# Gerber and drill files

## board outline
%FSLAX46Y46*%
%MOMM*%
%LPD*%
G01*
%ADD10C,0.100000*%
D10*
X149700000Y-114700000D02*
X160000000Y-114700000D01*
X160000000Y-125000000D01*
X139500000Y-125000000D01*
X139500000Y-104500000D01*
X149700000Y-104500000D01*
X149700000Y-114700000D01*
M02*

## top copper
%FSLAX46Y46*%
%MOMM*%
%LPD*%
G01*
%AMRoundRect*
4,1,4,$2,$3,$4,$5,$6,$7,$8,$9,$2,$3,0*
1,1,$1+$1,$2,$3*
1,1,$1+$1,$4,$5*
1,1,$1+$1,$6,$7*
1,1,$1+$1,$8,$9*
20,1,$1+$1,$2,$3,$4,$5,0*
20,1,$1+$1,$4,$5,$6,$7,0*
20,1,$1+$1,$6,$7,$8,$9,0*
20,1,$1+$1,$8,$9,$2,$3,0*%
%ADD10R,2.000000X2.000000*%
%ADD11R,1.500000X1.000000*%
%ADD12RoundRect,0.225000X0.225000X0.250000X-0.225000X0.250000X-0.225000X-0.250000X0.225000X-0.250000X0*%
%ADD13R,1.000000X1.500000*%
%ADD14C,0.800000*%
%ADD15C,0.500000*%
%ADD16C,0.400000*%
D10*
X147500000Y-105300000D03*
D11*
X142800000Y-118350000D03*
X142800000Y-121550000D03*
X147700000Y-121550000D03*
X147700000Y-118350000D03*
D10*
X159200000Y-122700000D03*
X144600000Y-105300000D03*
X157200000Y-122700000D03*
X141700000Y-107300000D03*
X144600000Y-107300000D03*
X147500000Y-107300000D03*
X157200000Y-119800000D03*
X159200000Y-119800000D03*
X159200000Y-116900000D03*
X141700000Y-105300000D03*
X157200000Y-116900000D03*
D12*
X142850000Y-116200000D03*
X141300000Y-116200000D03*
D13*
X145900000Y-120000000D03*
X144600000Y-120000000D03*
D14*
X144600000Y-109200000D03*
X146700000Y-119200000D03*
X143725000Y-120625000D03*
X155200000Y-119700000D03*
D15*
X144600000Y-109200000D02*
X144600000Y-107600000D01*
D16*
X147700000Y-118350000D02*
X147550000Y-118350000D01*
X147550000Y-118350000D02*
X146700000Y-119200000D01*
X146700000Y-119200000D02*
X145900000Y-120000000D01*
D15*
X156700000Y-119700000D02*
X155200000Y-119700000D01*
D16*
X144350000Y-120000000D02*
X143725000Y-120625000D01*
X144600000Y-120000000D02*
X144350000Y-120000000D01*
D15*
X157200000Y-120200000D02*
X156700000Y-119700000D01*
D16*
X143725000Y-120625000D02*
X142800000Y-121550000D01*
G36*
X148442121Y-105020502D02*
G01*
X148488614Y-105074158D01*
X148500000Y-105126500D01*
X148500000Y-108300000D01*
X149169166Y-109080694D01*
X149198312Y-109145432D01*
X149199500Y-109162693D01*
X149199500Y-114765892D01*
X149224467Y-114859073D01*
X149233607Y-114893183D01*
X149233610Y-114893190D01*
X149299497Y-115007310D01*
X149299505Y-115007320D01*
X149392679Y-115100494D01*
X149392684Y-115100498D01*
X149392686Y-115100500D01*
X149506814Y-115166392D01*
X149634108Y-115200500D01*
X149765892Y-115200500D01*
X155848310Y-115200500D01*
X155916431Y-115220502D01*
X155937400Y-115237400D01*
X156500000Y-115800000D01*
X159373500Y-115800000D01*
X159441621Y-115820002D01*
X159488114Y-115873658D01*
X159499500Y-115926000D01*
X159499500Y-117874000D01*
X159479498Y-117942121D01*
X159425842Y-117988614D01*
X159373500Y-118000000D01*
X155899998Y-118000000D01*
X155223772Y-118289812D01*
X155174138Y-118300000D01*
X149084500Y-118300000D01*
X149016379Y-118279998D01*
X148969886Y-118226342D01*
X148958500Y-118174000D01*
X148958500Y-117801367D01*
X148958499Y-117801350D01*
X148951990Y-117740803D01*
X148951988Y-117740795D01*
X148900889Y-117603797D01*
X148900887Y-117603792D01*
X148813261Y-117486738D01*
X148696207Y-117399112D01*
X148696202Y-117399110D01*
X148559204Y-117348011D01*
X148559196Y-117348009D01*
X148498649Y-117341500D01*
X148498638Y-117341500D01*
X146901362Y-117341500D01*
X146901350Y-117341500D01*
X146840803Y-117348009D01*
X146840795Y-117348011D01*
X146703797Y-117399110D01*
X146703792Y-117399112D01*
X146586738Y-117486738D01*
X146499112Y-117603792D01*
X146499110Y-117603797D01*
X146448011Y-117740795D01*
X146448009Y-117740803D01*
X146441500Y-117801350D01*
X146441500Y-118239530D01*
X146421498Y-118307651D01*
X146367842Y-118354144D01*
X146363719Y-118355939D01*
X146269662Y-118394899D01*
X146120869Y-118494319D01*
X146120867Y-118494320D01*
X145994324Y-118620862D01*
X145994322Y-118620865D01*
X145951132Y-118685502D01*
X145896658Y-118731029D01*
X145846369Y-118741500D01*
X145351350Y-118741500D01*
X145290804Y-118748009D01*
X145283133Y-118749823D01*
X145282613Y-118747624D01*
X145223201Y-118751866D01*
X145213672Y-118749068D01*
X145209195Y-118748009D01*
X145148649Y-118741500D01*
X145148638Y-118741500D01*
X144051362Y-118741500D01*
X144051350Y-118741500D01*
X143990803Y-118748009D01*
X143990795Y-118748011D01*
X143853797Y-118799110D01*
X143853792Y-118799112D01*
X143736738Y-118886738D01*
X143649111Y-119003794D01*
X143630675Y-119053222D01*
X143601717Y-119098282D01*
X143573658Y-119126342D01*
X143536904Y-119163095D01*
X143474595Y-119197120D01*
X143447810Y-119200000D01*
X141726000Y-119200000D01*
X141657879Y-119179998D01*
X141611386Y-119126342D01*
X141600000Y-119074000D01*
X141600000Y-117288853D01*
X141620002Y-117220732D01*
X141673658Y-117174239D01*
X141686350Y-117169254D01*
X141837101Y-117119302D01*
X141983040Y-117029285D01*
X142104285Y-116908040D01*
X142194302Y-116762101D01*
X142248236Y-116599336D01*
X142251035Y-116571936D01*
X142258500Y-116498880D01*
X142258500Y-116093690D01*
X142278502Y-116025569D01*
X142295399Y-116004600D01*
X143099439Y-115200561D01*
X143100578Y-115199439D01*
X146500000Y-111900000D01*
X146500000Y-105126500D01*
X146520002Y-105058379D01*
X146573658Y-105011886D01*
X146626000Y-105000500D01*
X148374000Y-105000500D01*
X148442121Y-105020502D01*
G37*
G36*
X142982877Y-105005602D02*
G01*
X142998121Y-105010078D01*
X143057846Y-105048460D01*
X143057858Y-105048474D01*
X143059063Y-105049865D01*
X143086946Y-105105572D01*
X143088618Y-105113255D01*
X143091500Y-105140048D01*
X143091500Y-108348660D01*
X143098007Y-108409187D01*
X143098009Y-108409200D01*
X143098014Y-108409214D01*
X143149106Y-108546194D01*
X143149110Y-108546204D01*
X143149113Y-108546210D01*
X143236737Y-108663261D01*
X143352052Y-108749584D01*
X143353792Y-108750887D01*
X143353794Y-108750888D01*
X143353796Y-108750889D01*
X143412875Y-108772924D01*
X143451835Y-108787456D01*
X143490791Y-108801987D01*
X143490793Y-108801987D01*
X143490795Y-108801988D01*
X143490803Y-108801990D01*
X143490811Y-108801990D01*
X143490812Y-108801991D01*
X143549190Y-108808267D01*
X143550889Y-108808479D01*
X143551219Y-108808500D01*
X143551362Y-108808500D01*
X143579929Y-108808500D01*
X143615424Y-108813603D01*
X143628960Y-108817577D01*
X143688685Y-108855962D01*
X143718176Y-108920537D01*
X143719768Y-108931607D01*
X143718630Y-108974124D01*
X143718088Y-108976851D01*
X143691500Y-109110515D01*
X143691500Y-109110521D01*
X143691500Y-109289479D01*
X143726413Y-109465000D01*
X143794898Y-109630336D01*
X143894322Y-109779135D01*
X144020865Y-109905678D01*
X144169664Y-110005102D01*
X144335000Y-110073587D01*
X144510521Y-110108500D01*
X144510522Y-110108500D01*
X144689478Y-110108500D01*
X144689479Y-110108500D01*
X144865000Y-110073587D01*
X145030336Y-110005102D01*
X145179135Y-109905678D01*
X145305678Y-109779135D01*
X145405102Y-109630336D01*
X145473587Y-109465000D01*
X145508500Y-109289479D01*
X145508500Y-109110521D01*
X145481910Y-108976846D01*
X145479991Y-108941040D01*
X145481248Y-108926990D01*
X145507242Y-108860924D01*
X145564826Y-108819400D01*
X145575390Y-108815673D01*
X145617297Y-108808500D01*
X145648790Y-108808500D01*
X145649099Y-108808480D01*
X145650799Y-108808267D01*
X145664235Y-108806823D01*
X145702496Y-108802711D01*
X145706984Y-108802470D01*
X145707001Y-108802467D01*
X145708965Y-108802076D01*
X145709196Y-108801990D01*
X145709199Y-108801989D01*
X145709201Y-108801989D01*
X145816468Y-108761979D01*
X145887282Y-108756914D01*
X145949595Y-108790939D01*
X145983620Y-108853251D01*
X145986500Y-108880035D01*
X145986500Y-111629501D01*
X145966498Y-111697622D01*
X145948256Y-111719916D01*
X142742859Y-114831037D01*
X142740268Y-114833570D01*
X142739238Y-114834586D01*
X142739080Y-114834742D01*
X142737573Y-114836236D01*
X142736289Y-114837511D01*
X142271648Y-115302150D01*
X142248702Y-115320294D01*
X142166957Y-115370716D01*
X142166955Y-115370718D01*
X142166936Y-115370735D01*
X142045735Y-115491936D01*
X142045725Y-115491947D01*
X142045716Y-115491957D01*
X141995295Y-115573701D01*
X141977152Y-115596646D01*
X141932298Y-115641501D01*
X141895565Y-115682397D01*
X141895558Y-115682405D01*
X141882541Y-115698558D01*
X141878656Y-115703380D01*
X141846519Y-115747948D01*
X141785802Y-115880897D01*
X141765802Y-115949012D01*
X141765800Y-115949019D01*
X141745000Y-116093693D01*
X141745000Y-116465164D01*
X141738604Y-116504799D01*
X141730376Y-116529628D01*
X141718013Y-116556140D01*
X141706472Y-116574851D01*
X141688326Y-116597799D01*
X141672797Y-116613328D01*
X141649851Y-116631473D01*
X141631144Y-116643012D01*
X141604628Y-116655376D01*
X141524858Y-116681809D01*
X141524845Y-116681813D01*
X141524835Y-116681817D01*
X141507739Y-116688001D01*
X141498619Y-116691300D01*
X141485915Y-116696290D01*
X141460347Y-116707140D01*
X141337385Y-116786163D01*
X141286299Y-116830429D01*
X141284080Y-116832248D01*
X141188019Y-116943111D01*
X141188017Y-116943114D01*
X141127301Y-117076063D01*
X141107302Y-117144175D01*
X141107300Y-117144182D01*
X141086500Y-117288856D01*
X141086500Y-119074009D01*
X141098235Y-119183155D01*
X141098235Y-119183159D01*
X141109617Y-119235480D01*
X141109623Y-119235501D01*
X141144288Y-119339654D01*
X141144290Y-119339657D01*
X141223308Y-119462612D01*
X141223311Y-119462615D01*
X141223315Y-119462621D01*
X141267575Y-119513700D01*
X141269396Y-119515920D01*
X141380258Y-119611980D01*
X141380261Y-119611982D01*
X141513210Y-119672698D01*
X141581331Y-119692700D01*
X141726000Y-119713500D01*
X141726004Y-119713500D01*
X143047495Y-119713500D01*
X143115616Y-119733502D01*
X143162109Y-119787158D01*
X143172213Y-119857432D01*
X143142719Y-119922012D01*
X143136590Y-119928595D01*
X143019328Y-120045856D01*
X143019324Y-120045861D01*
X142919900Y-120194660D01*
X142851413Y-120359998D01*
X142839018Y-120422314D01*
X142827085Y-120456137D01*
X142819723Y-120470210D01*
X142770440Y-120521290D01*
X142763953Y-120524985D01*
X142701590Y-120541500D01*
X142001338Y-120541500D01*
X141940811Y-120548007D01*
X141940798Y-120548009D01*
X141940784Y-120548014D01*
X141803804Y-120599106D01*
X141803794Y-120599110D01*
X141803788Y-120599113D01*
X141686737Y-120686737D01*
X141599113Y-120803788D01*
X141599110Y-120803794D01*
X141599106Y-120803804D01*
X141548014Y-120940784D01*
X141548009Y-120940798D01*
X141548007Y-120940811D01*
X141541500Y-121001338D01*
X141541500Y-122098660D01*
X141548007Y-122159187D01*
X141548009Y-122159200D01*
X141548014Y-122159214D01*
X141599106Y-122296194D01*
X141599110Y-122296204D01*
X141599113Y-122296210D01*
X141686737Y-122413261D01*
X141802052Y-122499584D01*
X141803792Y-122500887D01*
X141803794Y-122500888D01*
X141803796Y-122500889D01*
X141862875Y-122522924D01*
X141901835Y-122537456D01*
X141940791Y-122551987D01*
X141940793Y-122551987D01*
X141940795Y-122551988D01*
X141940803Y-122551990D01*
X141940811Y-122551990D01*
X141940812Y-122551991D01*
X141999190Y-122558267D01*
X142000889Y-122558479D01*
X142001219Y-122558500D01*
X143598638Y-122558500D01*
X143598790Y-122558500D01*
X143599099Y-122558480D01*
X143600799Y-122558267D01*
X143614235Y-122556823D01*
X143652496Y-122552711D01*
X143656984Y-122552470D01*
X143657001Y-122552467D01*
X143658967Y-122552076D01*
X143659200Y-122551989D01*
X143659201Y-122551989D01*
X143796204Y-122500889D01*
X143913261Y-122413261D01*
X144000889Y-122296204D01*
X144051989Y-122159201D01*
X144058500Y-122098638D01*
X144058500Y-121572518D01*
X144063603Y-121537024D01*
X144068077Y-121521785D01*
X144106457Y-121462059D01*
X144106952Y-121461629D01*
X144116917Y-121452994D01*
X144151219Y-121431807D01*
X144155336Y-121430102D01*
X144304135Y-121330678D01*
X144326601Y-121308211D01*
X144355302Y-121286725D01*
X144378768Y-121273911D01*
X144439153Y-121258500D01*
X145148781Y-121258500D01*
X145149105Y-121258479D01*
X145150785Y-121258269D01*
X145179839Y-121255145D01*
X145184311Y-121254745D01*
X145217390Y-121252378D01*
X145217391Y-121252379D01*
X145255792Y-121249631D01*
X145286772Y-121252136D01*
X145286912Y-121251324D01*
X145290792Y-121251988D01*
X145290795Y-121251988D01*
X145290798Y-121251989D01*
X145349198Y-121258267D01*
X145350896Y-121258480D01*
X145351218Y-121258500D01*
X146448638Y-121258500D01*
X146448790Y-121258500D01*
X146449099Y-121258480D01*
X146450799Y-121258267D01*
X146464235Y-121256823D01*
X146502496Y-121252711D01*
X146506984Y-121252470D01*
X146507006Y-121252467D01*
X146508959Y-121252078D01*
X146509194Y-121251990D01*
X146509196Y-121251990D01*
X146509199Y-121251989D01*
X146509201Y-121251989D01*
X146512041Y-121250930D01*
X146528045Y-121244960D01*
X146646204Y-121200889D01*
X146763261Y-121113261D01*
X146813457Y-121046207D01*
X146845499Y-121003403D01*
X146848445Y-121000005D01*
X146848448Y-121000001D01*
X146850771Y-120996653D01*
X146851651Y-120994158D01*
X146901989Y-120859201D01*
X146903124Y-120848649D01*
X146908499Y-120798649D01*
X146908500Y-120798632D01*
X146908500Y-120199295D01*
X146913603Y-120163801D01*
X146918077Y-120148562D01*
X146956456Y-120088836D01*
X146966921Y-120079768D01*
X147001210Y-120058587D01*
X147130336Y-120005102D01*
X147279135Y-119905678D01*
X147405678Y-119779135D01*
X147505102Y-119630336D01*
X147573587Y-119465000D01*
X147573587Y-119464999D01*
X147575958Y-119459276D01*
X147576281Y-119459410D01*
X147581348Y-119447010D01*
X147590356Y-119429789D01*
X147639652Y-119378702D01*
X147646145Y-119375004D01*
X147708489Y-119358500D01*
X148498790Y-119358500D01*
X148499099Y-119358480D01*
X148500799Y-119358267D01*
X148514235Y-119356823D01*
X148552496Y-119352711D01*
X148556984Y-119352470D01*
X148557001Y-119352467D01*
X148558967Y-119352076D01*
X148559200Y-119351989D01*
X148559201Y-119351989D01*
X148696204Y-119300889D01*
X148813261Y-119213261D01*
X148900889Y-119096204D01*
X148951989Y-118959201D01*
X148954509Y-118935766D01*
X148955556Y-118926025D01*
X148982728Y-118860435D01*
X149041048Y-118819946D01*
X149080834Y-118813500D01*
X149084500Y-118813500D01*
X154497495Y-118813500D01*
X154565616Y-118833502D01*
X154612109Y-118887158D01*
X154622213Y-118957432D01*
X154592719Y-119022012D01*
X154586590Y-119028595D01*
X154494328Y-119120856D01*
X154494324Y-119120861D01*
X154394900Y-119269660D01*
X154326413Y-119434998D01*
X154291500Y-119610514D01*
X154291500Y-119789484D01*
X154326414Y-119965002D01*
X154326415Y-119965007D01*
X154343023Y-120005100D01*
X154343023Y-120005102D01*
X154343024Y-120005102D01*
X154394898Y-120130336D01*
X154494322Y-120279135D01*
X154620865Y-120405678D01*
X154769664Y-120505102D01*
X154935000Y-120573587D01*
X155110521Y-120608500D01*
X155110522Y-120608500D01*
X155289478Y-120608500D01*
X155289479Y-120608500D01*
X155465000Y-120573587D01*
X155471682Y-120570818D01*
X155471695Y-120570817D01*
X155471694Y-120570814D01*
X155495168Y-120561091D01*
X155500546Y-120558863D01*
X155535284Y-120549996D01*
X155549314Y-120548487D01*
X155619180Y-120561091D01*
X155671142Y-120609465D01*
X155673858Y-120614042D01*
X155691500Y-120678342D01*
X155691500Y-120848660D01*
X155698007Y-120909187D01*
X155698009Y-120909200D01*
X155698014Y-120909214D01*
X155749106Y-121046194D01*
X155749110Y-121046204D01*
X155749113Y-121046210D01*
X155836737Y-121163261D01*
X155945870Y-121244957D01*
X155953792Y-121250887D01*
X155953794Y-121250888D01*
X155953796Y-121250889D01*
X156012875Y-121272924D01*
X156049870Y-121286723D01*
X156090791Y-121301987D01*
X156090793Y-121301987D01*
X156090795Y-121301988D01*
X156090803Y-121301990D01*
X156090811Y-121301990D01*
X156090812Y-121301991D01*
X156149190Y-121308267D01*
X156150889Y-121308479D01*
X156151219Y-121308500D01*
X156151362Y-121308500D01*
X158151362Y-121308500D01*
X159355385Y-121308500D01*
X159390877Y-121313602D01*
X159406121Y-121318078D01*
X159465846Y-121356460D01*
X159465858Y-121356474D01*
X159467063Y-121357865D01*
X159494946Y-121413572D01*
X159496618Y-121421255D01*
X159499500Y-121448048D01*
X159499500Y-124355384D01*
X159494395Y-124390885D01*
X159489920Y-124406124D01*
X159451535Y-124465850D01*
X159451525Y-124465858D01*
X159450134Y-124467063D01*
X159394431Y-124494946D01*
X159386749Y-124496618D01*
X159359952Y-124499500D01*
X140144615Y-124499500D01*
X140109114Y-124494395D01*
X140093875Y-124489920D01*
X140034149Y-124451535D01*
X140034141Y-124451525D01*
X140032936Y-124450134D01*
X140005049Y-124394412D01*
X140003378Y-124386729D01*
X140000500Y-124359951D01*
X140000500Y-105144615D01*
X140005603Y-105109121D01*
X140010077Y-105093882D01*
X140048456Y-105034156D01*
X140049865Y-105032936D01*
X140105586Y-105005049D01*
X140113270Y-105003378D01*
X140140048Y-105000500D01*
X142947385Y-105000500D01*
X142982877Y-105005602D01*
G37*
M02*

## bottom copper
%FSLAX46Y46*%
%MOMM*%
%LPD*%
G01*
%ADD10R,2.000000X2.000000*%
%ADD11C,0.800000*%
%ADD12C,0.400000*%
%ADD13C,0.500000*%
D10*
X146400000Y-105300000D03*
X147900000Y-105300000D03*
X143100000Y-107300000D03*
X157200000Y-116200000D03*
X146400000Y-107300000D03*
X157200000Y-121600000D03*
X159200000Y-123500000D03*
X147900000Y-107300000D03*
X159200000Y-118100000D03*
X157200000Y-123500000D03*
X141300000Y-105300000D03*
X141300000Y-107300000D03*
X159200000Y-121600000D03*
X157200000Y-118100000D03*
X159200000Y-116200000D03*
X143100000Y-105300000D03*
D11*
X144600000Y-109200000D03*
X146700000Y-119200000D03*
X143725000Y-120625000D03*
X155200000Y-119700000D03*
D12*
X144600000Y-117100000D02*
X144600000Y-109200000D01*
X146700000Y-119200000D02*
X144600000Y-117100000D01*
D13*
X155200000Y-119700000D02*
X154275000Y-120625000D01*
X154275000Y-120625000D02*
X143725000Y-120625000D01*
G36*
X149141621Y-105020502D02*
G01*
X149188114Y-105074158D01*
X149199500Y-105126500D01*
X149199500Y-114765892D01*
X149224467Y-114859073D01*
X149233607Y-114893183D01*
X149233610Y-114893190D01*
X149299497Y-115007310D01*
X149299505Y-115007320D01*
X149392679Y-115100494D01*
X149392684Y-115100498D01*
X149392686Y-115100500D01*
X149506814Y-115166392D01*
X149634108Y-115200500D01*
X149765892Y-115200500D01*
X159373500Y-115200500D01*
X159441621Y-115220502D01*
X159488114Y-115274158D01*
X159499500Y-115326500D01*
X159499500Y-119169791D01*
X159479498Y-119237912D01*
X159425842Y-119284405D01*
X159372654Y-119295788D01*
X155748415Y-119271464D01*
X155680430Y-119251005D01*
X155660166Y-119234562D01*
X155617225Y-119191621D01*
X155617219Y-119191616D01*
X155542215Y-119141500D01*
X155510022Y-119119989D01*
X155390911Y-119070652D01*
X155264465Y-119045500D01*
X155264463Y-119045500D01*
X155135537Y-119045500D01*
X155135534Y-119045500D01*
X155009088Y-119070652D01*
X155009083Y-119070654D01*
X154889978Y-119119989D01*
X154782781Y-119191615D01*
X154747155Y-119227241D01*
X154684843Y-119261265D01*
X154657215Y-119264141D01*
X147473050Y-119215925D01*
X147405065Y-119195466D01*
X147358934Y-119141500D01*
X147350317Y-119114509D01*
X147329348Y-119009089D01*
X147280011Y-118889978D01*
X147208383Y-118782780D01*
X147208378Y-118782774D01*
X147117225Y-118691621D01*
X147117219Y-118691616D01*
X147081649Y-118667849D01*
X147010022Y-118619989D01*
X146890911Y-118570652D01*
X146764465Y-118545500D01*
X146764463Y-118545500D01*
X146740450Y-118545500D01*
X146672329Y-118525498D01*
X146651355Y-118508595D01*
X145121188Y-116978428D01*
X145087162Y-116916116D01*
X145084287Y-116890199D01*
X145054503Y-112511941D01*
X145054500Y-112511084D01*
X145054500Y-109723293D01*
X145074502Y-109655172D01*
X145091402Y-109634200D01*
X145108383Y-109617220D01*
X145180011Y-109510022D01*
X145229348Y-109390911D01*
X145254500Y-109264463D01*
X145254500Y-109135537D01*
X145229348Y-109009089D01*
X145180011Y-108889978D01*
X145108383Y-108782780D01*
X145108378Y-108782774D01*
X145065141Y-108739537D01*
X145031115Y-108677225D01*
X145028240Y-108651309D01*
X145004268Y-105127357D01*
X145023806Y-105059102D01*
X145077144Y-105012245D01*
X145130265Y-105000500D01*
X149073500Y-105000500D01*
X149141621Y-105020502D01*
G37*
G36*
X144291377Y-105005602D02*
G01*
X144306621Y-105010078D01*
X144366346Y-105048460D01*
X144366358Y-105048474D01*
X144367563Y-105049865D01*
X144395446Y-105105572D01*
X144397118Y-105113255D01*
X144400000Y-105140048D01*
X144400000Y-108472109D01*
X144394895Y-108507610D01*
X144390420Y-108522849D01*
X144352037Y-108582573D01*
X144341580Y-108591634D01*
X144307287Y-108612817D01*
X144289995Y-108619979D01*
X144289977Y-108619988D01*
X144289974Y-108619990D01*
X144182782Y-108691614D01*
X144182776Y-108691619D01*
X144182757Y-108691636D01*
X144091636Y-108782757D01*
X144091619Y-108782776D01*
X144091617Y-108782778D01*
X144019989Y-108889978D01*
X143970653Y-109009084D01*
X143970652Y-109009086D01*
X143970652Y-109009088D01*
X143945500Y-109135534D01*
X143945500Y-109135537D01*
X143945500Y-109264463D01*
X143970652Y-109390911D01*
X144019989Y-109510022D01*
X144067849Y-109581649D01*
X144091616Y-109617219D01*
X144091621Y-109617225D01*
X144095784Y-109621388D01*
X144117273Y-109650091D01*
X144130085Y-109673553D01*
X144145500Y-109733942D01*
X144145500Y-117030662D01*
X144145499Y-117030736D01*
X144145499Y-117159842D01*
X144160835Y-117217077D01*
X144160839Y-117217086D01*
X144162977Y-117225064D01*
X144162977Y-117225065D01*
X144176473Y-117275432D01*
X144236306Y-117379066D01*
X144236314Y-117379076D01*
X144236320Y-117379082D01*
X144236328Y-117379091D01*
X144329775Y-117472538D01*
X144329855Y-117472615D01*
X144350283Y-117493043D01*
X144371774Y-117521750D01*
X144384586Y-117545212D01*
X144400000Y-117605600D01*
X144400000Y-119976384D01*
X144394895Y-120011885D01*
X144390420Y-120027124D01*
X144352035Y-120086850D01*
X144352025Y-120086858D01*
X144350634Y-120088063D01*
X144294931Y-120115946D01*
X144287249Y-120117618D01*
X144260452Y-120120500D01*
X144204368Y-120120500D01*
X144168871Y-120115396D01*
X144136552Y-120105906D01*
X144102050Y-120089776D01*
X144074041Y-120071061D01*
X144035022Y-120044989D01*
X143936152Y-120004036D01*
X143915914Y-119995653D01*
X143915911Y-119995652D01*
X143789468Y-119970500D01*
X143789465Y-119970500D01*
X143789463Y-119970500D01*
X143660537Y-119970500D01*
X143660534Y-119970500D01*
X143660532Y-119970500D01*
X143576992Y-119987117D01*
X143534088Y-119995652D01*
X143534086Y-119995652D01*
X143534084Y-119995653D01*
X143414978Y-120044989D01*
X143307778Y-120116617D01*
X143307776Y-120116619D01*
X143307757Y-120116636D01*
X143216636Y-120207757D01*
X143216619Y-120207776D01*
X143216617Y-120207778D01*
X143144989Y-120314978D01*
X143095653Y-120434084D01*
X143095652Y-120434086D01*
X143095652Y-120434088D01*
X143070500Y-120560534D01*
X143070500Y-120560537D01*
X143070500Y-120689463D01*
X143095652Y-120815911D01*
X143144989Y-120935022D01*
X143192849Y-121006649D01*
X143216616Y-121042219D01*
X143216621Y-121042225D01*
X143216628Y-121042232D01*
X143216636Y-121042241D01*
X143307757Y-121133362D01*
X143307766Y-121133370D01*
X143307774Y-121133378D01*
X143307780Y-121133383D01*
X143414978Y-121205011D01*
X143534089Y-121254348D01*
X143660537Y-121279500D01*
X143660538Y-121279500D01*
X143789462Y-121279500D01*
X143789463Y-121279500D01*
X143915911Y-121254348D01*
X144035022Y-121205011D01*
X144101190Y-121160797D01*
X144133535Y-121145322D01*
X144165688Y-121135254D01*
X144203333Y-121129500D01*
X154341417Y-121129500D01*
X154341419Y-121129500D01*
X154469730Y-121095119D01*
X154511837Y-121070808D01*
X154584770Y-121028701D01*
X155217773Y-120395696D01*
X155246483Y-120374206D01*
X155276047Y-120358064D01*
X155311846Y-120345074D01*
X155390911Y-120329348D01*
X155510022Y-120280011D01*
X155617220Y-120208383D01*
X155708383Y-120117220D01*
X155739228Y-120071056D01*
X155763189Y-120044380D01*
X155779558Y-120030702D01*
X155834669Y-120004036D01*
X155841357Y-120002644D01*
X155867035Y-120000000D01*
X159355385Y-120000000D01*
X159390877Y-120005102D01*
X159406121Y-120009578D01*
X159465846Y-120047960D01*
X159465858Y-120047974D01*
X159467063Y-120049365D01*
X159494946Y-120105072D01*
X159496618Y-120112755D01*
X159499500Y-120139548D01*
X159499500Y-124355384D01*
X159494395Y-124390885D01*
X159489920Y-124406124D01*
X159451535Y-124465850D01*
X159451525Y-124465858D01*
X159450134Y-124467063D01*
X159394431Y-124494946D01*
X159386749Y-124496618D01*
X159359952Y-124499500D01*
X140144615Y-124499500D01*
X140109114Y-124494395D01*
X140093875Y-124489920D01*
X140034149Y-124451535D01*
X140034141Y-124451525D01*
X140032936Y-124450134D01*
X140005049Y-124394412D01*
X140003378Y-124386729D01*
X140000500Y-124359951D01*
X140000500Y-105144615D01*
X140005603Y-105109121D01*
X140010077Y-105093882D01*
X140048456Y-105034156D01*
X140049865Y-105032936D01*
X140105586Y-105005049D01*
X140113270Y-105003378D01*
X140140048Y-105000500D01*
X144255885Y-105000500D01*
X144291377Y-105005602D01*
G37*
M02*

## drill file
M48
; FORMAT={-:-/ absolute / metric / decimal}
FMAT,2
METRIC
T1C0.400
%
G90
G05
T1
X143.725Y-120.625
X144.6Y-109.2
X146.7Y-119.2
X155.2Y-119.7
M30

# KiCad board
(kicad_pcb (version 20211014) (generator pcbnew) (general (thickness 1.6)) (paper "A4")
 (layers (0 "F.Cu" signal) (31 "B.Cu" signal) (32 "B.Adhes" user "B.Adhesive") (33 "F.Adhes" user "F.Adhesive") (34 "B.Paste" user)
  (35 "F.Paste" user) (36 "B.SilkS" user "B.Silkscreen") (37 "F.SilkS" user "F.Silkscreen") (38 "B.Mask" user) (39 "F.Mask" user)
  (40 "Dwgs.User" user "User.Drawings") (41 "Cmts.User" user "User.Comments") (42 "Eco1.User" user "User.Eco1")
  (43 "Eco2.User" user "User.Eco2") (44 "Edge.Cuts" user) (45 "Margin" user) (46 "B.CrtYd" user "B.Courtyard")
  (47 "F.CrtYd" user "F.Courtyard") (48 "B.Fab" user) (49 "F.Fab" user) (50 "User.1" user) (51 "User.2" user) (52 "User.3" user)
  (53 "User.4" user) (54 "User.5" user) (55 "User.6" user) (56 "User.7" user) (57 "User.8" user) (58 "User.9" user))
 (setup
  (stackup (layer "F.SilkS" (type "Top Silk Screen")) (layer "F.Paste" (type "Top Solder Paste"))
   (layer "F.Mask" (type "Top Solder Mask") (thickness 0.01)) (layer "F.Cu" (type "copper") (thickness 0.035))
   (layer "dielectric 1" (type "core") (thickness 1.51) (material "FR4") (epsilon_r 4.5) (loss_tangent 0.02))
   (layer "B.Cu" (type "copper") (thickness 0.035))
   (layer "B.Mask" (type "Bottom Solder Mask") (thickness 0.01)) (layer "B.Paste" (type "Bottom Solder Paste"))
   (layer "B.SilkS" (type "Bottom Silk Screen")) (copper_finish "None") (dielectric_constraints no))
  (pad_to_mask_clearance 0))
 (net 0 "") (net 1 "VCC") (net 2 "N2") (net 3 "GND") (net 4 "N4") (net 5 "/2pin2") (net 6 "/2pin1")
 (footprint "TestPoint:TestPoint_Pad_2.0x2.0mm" (layer "F.Cu") (at 147.5 105.3 180)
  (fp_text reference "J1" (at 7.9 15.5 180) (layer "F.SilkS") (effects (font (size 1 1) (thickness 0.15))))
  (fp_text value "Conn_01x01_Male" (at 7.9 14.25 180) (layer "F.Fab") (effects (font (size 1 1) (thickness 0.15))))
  (pad "1" smd rect locked (at 0 0 180) (size 2 2) (layers "F.Cu" "F.Mask") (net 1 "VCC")))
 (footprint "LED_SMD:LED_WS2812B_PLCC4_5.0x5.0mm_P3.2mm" (layer "F.Cu") (at 145.25 119.95)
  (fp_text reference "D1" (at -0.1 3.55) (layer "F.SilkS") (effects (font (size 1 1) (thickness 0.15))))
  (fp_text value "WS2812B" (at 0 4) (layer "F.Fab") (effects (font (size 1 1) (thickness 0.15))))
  (pad "1" smd rect locked (at -2.45 -1.6) (size 1.5 1) (layers "F.Cu" "F.Paste" "F.Mask") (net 1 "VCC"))
  (pad "2" smd rect locked (at -2.45 1.6) (size 1.5 1) (layers "F.Cu" "F.Paste" "F.Mask") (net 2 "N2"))
  (pad "3" smd rect locked (at 2.45 1.6) (size 1.5 1) (layers "F.Cu" "F.Paste" "F.Mask") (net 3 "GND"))
  (pad "4" smd rect locked (at 2.45 -1.6) (size 1.5 1) (layers "F.Cu" "F.Paste" "F.Mask") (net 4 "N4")))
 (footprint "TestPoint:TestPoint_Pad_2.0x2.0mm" (layer "F.Cu") (at 159.2 122.7 90)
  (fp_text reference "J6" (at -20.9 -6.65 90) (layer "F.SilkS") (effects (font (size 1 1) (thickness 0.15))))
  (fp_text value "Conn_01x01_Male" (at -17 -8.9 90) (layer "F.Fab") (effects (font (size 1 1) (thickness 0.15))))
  (pad "1" smd rect locked (at 0 0 90) (size 2 2) (layers "F.Cu" "F.Mask") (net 3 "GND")))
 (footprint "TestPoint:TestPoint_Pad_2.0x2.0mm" (layer "F.Cu") (at 144.6 105.3 180)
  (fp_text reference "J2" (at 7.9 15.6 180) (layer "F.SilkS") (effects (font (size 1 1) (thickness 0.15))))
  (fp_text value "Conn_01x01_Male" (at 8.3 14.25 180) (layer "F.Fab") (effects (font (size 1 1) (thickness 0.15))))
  (pad "1" smd rect locked (at 0 0 180) (size 2 2) (layers "F.Cu" "F.Mask") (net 4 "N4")))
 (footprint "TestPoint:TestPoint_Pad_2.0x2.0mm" (layer "F.Cu") (at 157.2 122.7 90)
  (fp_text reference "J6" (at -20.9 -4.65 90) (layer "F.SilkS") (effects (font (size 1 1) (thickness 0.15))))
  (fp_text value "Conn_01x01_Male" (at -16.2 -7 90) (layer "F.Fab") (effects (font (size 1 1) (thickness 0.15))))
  (pad "1" smd rect locked (at 0 0 90) (size 2 2) (layers "F.Cu" "F.Mask") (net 3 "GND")))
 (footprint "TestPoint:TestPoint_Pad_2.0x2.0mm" (layer "F.Cu") (at 141.7 107.3 180)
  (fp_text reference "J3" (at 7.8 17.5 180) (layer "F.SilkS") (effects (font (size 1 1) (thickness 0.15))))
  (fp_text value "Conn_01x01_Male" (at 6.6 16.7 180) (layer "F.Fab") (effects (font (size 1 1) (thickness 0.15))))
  (pad "1" smd rect locked (at 0 0 180) (size 2 2) (layers "F.Cu" "F.Mask") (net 3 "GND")))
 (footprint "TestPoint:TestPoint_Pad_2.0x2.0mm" (layer "F.Cu") (at 144.6 107.3 180)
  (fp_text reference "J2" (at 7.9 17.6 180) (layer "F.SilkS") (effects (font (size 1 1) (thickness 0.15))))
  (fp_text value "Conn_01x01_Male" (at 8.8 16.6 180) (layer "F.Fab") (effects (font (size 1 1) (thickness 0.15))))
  (pad "1" smd rect locked (at 0 0 180) (size 2 2) (layers "F.Cu" "F.Mask") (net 4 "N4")))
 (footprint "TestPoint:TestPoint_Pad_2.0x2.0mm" (layer "F.Cu") (at 147.5 107.3 180)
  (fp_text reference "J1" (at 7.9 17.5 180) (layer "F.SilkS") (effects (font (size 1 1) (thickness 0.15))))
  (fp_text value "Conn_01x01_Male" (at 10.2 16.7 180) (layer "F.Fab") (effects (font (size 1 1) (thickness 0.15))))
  (pad "1" smd rect locked (at 0 0 180) (size 2 2) (layers "F.Cu" "F.Mask") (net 1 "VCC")))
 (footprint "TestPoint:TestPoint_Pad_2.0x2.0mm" (layer "F.Cu") (at 157.2 119.8 90)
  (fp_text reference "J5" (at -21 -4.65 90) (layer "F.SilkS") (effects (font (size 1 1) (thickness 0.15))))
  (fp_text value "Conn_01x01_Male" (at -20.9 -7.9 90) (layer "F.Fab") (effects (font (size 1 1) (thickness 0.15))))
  (pad "1" smd rect locked (at 0 0 90) (size 2 2) (layers "F.Cu" "F.Mask") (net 2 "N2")))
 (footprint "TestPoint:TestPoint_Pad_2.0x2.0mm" (layer "F.Cu") (at 159.2 119.8 90)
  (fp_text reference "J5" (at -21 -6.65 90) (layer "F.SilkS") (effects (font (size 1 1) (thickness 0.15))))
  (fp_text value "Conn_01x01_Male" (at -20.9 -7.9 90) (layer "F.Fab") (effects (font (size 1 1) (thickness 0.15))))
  (pad "1" smd rect locked (at 0 0 90) (size 2 2) (layers "F.Cu" "F.Mask") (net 2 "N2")))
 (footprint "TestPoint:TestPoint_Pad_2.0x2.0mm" (layer "F.Cu") (at 159.2 116.9 90)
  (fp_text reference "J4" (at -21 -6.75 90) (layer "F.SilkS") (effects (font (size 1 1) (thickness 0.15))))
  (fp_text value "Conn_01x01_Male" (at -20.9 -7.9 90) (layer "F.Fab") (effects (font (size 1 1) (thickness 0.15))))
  (pad "1" smd rect locked (at 0 0 90) (size 2 2) (layers "F.Cu" "F.Mask") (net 1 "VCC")))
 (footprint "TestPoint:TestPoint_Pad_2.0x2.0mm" (layer "F.Cu") (at 141.7 105.3 180)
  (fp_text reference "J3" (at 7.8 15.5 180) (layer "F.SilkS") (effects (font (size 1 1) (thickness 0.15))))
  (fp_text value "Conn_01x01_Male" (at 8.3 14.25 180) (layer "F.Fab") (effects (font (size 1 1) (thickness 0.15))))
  (pad "1" smd rect locked (at 0 0 180) (size 2 2) (layers "F.Cu" "F.Mask") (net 3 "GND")))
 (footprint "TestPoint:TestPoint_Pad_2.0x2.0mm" (layer "F.Cu") (at 157.2 116.9 90)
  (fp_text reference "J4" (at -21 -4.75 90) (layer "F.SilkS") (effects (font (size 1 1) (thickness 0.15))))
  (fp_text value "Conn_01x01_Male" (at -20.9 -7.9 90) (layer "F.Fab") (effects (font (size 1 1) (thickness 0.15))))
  (pad "1" smd rect locked (at 0 0 90) (size 2 2) (layers "F.Cu" "F.Mask") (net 1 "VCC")))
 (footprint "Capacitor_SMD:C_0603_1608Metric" (layer "F.Cu") (at 142.075 116.2 180)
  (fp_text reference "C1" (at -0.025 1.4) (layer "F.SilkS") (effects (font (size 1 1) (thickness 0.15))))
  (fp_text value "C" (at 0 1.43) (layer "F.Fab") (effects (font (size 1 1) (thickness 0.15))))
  (pad "1" smd roundrect locked (at -0.775 0 180) (size 0.9 0.95) (layers "F.Cu" "F.Paste" "F.Mask") (roundrect_rratio 0.25) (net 1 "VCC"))
  (pad "2" smd roundrect locked (at 0.775 0 180) (size 0.9 0.95) (layers "F.Cu" "F.Paste" "F.Mask") (roundrect_rratio 0.25) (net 3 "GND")))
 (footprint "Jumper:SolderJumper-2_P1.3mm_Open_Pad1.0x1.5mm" (layer "F.Cu") (at 145.25 120 180)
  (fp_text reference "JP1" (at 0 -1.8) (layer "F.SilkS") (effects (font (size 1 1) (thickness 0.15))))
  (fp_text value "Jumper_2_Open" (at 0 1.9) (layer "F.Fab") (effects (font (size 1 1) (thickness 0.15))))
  (pad "1" smd rect locked (at -0.65 0 180) (size 1 1.5) (layers "F.Cu" "F.Mask") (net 4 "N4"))
  (pad "2" smd rect locked (at 0.65 0 180) (size 1 1.5) (layers "F.Cu" "F.Mask") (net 2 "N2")))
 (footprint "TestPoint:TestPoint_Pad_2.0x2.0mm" (layer "B.Cu") (at 146.4 105.3 180)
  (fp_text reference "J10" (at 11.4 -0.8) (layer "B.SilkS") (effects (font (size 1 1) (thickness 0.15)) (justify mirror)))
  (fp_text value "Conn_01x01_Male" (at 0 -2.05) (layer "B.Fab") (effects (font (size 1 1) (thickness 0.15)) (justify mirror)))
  (pad "1" smd rect (at 0 0 180) (size 2 2) (layers "B.Cu" "B.Mask") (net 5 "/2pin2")))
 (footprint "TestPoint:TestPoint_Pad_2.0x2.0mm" (layer "B.Cu") (at 147.9 105.3 180)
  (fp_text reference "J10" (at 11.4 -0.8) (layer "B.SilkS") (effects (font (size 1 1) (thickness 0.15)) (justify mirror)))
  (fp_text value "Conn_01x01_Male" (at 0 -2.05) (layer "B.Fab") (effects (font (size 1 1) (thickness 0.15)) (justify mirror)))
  (pad "1" smd rect (at 0 0 180) (size 2 2) (layers "B.Cu" "B.Mask") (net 5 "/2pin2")))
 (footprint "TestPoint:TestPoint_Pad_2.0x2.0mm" (layer "B.Cu") (at 143.1 107.3 180)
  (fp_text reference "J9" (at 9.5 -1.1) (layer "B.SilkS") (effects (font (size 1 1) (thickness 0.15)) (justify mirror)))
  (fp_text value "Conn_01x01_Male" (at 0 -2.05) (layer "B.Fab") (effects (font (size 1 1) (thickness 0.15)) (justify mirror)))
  (pad "1" smd rect (at 0 0 180) (size 2 2) (layers "B.Cu" "B.Mask") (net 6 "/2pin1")))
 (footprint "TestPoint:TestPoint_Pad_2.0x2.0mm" (layer "B.Cu") (at 157.2 116.2 180)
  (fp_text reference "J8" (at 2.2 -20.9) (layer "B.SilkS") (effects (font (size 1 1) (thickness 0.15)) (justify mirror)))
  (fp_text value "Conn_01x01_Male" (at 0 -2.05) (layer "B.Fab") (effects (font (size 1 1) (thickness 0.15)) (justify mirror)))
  (pad "1" smd rect (at 0 0 180) (size 2 2) (layers "B.Cu" "B.Mask") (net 5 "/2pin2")))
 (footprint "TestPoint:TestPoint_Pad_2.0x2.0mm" (layer "B.Cu") (at 146.4 107.3 180)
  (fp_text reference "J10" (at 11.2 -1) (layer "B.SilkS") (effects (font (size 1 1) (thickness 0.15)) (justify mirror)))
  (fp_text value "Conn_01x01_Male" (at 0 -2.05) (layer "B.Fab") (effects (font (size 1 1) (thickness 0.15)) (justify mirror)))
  (pad "1" smd rect (at 0 0 180) (size 2 2) (layers "B.Cu" "B.Mask") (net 5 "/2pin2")))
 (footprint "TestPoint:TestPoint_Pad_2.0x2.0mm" (layer "B.Cu") (at 157.2 121.6 180)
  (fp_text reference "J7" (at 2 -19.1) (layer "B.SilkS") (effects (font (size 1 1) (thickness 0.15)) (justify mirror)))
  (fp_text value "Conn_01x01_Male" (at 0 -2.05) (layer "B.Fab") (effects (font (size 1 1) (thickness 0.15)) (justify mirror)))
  (pad "1" smd rect (at 0 0 180) (size 2 2) (layers "B.Cu" "B.Mask") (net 6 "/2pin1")))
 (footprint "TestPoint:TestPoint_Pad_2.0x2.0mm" (layer "B.Cu") (at 159.2 123.5 180)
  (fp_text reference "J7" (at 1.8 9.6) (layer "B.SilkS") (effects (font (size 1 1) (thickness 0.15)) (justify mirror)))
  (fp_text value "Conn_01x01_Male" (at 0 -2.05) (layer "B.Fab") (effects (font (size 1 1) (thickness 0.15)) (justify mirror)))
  (pad "1" smd rect (at 0 0 180) (size 2 2) (layers "B.Cu" "B.Mask") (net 6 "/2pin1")))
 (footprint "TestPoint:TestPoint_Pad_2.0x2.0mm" (layer "B.Cu") (at 147.9 107.3 180)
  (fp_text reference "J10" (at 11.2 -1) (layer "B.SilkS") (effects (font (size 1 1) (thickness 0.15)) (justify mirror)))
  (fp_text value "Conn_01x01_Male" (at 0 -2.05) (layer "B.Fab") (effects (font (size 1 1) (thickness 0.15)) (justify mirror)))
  (pad "1" smd rect (at 0 0 180) (size 2 2) (layers "B.Cu" "B.Mask") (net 5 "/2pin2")))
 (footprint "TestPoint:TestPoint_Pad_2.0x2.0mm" (layer "B.Cu") (at 159.2 118.1 180)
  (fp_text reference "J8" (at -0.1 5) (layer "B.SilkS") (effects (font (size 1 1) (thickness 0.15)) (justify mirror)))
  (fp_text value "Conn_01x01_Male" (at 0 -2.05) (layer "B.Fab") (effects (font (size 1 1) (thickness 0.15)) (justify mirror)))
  (pad "1" smd rect (at 0 0 180) (size 2 2) (layers "B.Cu" "B.Mask") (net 5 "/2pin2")))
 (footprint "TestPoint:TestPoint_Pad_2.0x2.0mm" (layer "B.Cu") (at 157.2 123.5 180)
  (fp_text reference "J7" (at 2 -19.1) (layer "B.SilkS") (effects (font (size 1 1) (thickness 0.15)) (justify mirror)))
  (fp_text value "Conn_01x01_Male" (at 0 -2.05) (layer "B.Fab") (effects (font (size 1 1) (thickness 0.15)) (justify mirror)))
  (pad "1" smd rect (at 0 0 180) (size 2 2) (layers "B.Cu" "B.Mask") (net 6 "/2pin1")))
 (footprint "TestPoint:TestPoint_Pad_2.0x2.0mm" (layer "B.Cu") (at 141.3 105.3 180)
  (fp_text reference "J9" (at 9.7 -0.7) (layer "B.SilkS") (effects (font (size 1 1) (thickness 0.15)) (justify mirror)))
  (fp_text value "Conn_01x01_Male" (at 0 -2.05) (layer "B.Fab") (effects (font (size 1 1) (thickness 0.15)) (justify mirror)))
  (pad "1" smd rect (at 0 0 180) (size 2 2) (layers "B.Cu" "B.Mask") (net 6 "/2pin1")))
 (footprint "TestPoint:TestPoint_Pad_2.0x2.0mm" (layer "B.Cu") (at 141.3 107.3 180)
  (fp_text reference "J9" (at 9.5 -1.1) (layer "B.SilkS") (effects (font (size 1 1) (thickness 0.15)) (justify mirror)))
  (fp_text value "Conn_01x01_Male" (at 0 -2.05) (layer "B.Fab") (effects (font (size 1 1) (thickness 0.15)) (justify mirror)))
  (pad "1" smd rect (at 0 0 180) (size 2 2) (layers "B.Cu" "B.Mask") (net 6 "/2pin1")))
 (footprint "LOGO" (layer "B.Cu") (at 144.75 119.75 180)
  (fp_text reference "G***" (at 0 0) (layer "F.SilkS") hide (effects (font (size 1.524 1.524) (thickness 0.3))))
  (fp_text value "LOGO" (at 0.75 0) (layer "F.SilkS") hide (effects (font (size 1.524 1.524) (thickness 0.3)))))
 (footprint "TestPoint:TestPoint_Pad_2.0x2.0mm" (layer "B.Cu") (at 159.2 121.6 180)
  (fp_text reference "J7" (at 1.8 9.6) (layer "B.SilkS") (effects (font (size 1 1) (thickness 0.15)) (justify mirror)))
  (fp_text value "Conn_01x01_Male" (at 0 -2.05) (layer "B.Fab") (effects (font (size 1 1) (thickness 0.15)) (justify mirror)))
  (pad "1" smd rect (at 0 0 180) (size 2 2) (layers "B.Cu" "B.Mask") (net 6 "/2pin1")))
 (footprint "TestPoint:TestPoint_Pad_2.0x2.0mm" (layer "B.Cu") (at 157.2 118.1 180)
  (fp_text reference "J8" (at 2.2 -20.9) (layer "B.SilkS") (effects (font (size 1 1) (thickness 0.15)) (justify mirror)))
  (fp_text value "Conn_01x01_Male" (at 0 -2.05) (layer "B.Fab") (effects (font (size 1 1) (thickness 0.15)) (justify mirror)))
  (pad "1" smd rect (at 0 0 180) (size 2 2) (layers "B.Cu" "B.Mask") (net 5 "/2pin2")))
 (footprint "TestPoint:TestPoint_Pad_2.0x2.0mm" (layer "B.Cu") (at 159.2 116.2 180)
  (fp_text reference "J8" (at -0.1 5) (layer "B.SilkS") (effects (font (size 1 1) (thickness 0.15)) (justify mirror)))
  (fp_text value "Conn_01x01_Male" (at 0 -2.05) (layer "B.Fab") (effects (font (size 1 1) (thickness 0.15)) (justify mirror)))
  (pad "1" smd rect (at 0 0 180) (size 2 2) (layers "B.Cu" "B.Mask") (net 5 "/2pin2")))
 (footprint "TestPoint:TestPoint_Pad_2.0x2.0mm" (layer "B.Cu") (at 143.1 105.3 180)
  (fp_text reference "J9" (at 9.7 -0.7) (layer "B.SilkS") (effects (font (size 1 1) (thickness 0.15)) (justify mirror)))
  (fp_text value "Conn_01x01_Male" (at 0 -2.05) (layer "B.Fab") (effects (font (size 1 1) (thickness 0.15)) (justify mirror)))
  (pad "1" smd rect (at 0 0 180) (size 2 2) (layers "B.Cu" "B.Mask") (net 6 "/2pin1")))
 (gr_poly
  (pts (xy 149.7 114.7) (xy 160 114.7) (xy 160 125) (xy 139.5 125) (xy 139.5 104.5) (xy 149.7 104.5)) (layer "Edge.Cuts") (width 0.1)
  (fill none))
 (segment (start 144.6 109.2) (end 144.6 107.6) (width 0.5) (layer "F.Cu") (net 4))
 (segment (start 147.7 118.35) (end 147.55 118.35) (width 0.4) (layer "F.Cu") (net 4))
 (segment (start 147.55 118.35) (end 146.7 119.2) (width 0.4) (layer "F.Cu") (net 4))
 (segment (start 146.7 119.2) (end 145.9 120) (width 0.4) (layer "F.Cu") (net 4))
 (via (at 144.6 109.2) (size 0.8) (drill 0.4) (layers "F.Cu" "B.Cu") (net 4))
 (via (at 146.7 119.2) (size 0.8) (drill 0.4) (layers "F.Cu" "B.Cu") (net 4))
 (segment (start 144.6 117.1) (end 144.6 109.2) (width 0.4) (layer "B.Cu") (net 4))
 (segment (start 146.7 119.2) (end 144.6 117.1) (width 0.4) (layer "B.Cu") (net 4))
 (segment (start 156.7 119.7) (end 155.2 119.7) (width 0.5) (layer "F.Cu") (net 2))
 (segment (start 144.35 120) (end 143.725 120.625) (width 0.4) (layer "F.Cu") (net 2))
 (segment (start 144.6 120) (end 144.35 120) (width 0.4) (layer "F.Cu") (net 2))
 (segment (start 157.2 120.2) (end 156.7 119.7) (width 0.5) (layer "F.Cu") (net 2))
 (segment (start 143.725 120.625) (end 142.8 121.55) (width 0.4) (layer "F.Cu") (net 2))
 (via (at 143.725 120.625) (size 0.8) (drill 0.4) (layers "F.Cu" "B.Cu") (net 2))
 (via (at 155.2 119.7) (size 0.8) (drill 0.4) (layers "F.Cu" "B.Cu") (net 2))
 (segment (start 155.2 119.7) (end 154.275 120.625) (width 0.5) (layer "B.Cu") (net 2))
 (segment (start 154.275 120.625) (end 143.725 120.625) (width 0.5) (layer "B.Cu") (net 2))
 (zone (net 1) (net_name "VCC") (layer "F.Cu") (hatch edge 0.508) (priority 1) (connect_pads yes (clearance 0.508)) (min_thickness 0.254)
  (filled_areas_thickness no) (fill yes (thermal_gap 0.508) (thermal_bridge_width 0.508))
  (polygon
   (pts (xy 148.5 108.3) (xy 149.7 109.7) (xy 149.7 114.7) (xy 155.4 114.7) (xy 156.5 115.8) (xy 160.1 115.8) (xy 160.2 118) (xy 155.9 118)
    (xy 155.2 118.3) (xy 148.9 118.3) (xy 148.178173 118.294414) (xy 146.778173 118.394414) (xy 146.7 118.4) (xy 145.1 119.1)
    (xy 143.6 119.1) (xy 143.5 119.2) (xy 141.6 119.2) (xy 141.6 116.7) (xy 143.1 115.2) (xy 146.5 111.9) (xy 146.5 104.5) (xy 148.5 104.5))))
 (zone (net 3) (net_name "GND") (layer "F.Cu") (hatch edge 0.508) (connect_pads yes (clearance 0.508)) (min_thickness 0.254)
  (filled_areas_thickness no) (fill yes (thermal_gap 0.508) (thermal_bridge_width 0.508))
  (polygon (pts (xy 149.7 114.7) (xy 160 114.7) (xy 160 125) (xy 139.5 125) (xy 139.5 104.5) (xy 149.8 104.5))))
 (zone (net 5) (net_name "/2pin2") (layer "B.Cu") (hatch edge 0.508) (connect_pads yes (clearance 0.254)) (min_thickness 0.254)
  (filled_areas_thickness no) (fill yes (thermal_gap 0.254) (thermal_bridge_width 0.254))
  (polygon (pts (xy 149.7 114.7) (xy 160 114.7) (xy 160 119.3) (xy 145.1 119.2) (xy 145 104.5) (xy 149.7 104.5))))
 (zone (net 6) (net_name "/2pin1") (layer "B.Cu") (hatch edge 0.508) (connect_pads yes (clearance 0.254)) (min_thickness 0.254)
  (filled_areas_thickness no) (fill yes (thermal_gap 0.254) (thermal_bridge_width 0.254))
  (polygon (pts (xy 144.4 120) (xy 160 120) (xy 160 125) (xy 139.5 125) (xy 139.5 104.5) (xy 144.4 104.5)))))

